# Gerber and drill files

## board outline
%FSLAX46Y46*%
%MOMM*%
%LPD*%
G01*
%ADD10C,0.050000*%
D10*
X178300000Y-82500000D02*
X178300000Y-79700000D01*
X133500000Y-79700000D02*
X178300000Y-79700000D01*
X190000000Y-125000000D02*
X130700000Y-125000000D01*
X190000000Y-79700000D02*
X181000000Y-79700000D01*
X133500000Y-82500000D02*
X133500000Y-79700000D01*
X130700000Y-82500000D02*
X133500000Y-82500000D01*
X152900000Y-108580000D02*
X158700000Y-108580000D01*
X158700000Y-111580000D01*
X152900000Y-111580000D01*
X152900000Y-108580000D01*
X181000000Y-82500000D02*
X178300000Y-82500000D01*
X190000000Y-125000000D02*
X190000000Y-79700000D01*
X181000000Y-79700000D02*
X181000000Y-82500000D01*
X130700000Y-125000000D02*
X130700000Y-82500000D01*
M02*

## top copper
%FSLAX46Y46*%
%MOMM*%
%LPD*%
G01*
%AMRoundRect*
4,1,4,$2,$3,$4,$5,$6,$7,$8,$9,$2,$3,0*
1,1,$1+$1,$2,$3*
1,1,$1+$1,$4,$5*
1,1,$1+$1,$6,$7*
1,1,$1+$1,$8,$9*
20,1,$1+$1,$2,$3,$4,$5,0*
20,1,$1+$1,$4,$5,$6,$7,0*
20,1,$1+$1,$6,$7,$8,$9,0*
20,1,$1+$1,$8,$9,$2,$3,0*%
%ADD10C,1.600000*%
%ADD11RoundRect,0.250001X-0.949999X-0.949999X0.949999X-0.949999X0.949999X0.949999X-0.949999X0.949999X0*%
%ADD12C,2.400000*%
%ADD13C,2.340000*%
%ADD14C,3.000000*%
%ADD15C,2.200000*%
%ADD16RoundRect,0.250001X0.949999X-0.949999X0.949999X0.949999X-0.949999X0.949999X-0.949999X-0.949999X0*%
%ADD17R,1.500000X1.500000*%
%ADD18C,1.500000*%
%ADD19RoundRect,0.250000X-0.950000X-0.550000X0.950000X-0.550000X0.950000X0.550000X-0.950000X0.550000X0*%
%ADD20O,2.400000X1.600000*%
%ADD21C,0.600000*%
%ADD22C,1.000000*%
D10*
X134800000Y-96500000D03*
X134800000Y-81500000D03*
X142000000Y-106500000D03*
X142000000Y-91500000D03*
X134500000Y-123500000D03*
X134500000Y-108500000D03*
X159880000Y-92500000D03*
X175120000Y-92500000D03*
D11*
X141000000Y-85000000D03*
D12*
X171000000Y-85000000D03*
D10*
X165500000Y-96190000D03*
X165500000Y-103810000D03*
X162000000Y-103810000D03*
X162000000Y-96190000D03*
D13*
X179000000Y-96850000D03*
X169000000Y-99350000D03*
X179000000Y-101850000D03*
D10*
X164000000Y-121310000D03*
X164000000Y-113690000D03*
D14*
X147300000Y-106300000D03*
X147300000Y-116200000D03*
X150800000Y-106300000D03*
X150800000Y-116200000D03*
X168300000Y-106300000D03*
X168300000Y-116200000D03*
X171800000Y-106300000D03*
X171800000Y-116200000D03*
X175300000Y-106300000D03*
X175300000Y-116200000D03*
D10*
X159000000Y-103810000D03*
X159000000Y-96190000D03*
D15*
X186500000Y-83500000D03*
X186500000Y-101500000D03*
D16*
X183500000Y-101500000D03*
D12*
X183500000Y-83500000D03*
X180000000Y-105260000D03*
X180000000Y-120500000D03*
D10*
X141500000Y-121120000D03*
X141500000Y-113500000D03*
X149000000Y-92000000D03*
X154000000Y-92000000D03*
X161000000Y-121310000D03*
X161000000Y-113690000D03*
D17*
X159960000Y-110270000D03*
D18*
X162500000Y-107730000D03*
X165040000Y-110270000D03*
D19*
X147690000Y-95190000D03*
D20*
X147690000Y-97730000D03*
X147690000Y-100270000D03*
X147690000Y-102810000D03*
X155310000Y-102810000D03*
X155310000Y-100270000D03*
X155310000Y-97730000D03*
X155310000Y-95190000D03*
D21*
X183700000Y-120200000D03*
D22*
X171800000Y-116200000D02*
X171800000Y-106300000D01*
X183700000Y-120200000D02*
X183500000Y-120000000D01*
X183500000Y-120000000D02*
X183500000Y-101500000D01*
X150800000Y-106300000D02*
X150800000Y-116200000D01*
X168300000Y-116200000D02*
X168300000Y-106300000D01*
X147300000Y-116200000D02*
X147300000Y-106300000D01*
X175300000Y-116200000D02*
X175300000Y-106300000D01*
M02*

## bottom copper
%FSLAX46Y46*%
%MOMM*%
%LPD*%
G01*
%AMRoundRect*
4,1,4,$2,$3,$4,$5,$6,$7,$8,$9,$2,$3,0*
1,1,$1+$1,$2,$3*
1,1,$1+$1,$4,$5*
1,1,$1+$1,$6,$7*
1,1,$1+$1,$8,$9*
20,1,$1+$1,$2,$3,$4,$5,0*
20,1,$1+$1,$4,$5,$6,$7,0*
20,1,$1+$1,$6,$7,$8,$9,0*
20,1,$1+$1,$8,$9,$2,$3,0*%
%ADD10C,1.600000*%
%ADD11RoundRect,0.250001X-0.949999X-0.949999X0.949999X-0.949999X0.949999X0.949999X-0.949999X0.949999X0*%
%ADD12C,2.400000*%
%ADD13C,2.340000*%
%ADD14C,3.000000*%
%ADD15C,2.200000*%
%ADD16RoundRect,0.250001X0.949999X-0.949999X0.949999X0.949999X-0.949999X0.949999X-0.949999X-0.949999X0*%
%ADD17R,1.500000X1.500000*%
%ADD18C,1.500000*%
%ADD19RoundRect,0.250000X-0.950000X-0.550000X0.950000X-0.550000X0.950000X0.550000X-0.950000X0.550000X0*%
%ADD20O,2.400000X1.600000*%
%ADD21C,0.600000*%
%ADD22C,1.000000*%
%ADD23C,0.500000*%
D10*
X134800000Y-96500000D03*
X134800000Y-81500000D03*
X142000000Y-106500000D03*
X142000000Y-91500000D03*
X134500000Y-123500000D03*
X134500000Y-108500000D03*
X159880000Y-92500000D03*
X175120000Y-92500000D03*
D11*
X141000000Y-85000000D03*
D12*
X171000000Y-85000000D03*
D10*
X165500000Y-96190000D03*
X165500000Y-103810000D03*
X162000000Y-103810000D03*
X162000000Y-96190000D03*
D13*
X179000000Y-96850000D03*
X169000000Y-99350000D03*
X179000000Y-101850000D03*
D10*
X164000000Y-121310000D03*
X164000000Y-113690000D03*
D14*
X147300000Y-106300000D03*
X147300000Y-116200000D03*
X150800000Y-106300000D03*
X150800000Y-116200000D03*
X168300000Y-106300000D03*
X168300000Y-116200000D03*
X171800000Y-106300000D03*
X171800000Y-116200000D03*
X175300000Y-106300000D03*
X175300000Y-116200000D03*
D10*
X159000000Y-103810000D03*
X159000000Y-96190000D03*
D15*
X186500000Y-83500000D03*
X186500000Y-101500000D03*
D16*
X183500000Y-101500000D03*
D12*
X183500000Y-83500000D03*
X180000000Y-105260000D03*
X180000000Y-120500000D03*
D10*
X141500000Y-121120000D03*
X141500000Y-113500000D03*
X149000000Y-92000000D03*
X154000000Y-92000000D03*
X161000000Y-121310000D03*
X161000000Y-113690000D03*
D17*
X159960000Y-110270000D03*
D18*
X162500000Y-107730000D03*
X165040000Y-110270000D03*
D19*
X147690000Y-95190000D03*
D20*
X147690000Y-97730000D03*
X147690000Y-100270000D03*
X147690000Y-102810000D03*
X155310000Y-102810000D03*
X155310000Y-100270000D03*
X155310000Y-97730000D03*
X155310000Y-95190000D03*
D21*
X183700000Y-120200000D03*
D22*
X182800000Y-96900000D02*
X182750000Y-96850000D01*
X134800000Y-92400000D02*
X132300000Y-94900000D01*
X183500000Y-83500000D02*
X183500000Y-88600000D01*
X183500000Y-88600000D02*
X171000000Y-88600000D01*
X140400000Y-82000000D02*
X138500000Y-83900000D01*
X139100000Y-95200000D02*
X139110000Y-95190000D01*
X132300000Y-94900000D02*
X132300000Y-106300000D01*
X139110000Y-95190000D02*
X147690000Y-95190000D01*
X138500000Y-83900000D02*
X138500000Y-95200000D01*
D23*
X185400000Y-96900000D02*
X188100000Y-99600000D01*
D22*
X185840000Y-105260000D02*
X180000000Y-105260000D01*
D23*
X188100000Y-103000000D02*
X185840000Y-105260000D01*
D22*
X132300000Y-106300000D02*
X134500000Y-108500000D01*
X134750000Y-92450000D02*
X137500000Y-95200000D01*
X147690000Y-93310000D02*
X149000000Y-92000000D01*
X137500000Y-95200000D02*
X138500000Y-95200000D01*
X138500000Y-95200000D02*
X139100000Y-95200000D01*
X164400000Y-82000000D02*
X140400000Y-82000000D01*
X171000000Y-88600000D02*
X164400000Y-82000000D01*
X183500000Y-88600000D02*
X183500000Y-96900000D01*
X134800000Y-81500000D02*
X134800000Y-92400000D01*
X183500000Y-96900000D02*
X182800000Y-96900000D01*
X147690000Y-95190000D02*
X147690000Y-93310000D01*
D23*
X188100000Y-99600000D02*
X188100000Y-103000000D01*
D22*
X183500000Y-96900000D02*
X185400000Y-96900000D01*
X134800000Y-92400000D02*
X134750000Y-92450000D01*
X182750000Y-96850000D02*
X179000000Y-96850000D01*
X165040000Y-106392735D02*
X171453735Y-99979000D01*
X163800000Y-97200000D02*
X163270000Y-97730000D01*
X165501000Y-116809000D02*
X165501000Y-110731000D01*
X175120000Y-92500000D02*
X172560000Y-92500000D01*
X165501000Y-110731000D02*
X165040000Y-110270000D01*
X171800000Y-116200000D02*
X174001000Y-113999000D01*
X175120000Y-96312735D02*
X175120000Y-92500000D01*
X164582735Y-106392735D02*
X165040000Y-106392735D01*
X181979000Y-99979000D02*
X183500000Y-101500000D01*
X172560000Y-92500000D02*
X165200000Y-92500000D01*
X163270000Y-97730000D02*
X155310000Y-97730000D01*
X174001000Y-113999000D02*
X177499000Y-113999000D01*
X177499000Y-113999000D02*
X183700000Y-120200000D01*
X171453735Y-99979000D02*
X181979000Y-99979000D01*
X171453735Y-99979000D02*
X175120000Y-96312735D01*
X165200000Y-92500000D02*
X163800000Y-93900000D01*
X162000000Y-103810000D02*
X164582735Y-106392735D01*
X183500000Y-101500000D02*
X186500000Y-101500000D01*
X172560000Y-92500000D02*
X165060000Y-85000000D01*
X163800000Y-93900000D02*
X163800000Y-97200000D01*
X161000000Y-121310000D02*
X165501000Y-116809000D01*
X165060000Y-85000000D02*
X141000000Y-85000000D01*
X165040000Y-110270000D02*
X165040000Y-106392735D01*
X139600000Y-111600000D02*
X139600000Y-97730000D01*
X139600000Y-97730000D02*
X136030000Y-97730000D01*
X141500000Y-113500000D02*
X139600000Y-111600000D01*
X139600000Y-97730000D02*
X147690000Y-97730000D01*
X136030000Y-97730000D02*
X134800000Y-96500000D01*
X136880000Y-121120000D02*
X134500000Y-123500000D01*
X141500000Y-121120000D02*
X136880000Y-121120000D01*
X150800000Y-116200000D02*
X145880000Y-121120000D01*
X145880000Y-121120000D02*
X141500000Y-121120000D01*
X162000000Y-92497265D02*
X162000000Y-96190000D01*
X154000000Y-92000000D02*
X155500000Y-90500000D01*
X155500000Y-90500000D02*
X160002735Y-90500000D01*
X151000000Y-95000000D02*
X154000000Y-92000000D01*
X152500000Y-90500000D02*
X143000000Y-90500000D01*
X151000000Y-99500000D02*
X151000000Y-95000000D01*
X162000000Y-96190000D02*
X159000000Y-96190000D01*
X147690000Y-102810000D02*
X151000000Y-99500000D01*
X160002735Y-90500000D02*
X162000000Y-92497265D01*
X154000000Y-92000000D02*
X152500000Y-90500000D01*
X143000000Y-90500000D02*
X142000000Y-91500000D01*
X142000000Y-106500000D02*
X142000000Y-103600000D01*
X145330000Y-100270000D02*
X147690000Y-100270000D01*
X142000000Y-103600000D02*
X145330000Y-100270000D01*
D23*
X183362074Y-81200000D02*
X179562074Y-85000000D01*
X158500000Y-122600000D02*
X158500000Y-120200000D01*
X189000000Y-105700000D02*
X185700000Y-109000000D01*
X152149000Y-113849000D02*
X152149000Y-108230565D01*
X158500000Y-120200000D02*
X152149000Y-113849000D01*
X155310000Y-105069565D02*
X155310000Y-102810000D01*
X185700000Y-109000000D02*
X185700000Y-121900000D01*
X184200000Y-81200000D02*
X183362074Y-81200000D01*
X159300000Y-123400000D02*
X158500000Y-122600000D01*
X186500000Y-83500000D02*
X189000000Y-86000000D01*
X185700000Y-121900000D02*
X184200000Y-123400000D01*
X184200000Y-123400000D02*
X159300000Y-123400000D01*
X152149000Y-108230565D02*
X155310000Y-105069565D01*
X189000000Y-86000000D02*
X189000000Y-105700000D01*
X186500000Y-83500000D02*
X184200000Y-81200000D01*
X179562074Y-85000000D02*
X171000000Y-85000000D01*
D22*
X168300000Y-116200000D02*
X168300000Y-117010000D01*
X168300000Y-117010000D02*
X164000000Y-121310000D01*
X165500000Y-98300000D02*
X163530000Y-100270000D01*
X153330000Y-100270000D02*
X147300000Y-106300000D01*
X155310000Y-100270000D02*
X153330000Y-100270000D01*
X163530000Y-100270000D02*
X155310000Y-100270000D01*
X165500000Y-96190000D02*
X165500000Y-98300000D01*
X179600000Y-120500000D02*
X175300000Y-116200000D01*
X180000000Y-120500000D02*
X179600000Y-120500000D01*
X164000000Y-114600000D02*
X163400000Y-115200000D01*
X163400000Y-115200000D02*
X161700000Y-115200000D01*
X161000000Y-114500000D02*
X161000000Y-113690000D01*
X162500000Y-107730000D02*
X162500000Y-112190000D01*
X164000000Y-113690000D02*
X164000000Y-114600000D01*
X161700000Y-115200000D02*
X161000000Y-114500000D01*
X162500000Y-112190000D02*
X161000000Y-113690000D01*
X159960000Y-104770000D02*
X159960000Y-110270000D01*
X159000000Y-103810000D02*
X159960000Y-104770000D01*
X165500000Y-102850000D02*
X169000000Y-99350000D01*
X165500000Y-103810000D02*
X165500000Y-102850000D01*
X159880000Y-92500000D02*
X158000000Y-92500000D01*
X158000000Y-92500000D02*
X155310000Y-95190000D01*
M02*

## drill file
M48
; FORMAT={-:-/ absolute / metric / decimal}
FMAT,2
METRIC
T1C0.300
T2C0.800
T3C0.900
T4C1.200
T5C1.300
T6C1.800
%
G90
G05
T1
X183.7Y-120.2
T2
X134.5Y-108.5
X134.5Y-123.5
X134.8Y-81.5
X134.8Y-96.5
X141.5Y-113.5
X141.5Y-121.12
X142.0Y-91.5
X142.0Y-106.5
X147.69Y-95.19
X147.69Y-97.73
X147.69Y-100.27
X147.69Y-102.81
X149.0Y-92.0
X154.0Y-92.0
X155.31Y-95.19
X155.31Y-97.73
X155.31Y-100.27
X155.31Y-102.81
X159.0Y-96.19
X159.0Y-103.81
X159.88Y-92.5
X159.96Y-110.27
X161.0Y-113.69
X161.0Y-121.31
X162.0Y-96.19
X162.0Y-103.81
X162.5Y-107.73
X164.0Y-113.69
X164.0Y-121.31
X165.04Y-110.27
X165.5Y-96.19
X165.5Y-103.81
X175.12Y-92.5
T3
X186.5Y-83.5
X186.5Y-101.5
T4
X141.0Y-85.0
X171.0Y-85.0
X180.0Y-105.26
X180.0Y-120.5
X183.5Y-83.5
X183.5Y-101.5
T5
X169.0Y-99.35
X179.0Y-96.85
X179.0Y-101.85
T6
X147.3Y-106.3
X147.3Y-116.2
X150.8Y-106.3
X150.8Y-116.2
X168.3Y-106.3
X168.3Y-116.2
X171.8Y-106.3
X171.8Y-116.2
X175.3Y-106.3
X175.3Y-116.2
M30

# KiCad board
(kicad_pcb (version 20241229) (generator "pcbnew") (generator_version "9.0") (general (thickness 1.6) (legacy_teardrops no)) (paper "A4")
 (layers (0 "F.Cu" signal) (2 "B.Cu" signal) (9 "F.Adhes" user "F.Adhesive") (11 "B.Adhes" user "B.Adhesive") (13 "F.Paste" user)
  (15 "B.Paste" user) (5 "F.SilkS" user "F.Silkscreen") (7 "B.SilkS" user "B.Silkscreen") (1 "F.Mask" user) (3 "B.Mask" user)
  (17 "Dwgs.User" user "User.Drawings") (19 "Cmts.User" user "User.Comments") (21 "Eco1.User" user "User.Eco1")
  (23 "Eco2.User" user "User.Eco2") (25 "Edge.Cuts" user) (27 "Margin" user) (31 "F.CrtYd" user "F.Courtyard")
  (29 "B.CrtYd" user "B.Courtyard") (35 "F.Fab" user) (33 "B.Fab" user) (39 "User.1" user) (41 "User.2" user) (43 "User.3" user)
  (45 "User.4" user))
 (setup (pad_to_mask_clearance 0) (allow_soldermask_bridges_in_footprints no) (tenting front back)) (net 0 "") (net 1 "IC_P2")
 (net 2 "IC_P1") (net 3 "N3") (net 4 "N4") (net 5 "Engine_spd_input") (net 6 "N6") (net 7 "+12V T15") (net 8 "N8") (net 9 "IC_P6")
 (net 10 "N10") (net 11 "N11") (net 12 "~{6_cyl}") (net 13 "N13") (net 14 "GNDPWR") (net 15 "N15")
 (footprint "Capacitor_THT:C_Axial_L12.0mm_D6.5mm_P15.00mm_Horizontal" (layer "F.Cu") (at 134.8 96.5 90)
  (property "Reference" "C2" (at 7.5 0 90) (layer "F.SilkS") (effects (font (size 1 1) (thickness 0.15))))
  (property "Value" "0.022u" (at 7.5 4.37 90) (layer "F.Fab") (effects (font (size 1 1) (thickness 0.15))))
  (pad "1" thru_hole circle (at 0 0 90) (size 1.6 1.6) (drill 0.8) (layers "*.Cu" "*.Mask") (remove_unused_layers no) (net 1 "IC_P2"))
  (pad "2" thru_hole circle (at 15 0 90) (size 1.6 1.6) (drill 0.8) (layers "*.Cu" "*.Mask") (remove_unused_layers no) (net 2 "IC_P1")))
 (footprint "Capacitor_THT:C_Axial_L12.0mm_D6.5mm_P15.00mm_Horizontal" (layer "F.Cu") (at 142 106.5 90)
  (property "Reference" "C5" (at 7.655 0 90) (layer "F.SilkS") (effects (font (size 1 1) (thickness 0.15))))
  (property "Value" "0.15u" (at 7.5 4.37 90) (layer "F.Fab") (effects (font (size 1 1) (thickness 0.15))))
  (pad "1" thru_hole circle (at 0 0 90) (size 1.6 1.6) (drill 0.8) (layers "*.Cu" "*.Mask") (remove_unused_layers no) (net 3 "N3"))
  (pad "2" thru_hole circle (at 15 0 90) (size 1.6 1.6) (drill 0.8) (layers "*.Cu" "*.Mask") (remove_unused_layers no) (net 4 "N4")))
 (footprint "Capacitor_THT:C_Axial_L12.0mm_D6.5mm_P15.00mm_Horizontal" (layer "F.Cu") (at 134.5 123.5 90)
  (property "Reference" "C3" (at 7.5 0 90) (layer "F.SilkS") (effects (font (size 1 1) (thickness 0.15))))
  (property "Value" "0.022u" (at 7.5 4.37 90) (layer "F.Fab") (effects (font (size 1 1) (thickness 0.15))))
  (pad "1" thru_hole circle (at 0 0 90) (size 1.6 1.6) (drill 0.8) (layers "*.Cu" "*.Mask") (remove_unused_layers no)
   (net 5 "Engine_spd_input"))
  (pad "2" thru_hole circle (at 15 0 90) (size 1.6 1.6) (drill 0.8) (layers "*.Cu" "*.Mask") (remove_unused_layers no) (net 2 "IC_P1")))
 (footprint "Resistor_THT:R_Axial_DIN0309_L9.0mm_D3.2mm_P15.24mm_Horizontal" (layer "F.Cu") (at 159.88 92.5)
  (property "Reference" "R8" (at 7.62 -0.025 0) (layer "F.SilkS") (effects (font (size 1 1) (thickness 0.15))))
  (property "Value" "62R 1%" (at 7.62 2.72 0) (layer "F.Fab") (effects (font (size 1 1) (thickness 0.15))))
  (pad "1" thru_hole circle (at 0 0) (size 1.6 1.6) (drill 0.8) (layers "*.Cu" "*.Mask") (remove_unused_layers no) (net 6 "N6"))
  (pad "2" thru_hole circle (at 15.24 0) (size 1.6 1.6) (drill 0.8) (layers "*.Cu" "*.Mask") (remove_unused_layers no) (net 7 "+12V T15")))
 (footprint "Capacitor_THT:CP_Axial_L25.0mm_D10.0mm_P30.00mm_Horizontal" (layer "F.Cu") (at 141 85)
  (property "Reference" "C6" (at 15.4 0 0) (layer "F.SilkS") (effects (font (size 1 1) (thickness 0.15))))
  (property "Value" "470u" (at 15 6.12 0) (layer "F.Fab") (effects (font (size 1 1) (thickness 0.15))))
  (pad "1" thru_hole roundrect (at 0 0) (size 2.4 2.4) (drill 1.2) (layers "*.Cu" "*.Mask") (remove_unused_layers no)
   (roundrect_rratio 0.104167) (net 7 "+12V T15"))
  (pad "2" thru_hole circle (at 30 0) (size 2.4 2.4) (drill 1.2) (layers "*.Cu" "*.Mask") (remove_unused_layers no) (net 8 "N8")))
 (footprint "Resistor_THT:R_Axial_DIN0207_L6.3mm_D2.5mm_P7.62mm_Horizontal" (layer "F.Cu") (at 165.5 96.19 -90)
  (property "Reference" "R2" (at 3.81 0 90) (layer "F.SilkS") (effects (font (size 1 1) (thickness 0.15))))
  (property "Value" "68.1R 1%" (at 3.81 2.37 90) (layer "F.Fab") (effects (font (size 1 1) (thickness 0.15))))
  (pad "1" thru_hole circle (at 0 0 270) (size 1.6 1.6) (drill 0.8) (layers "*.Cu" "*.Mask") (remove_unused_layers no) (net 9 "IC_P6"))
  (pad "2" thru_hole circle (at 7.62 0 270) (size 1.6 1.6) (drill 0.8) (layers "*.Cu" "*.Mask") (remove_unused_layers no) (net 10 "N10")))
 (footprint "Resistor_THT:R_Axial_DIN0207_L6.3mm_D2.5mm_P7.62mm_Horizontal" (layer "F.Cu") (at 162 103.81 90)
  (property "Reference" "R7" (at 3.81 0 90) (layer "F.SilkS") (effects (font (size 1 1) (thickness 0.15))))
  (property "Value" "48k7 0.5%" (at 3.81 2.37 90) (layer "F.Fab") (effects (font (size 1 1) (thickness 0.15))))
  (pad "1" thru_hole circle (at 0 0 90) (size 1.6 1.6) (drill 0.8) (layers "*.Cu" "*.Mask") (remove_unused_layers no) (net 7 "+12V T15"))
  (pad "2" thru_hole circle (at 7.62 0 90) (size 1.6 1.6) (drill 0.8) (layers "*.Cu" "*.Mask") (remove_unused_layers no) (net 4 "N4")))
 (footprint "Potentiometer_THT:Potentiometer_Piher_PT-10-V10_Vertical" (layer "F.Cu") (at 179 96.85 180)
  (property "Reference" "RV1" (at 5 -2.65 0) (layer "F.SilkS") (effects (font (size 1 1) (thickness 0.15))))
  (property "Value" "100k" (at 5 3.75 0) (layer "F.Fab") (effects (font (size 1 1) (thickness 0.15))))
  (pad "1" thru_hole circle (at 0 0 180) (size 2.34 2.34) (drill 1.3) (layers "*.Cu" "*.Mask") (remove_unused_layers no) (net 2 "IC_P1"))
  (pad "2" thru_hole circle (at 10 -2.5 180) (size 2.34 2.34) (drill 1.3) (layers "*.Cu" "*.Mask") (remove_unused_layers no) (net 10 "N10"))
  (pad "3" thru_hole circle (at 0 -5 180) (size 2.34 2.34) (drill 1.3) (layers "*.Cu" "*.Mask") (remove_unused_layers no) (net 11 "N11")))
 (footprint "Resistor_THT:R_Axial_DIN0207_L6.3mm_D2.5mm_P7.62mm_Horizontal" (layer "F.Cu") (at 164 121.31 90)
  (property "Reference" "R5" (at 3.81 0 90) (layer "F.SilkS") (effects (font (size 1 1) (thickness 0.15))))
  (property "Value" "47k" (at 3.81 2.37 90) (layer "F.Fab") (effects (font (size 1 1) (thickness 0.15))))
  (pad "1" thru_hole circle (at 0 0 90) (size 1.6 1.6) (drill 0.8) (layers "*.Cu" "*.Mask") (remove_unused_layers no) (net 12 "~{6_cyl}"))
  (pad "2" thru_hole circle (at 7.62 0 90) (size 1.6 1.6) (drill 0.8) (layers "*.Cu" "*.Mask") (remove_unused_layers no) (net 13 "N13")))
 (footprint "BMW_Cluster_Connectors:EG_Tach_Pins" (layer "F.Cu") (at 147.3 106.3)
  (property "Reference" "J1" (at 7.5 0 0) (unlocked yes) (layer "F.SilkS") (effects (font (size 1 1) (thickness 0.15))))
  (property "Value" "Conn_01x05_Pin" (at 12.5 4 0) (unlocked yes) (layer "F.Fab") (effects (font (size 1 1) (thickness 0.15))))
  (pad "1" thru_hole circle (at 0 0 270) (size 3 3) (drill 1.8) (layers "*.Cu" "*.Mask") (remove_unused_layers no) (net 9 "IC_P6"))
  (pad "1" thru_hole circle (at 0 9.9 270) (size 3 3) (drill 1.8) (layers "*.Cu" "*.Mask") (remove_unused_layers no) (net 9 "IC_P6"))
  (pad "2" thru_hole circle (at 3.5 0 270) (size 3 3) (drill 1.8) (layers "*.Cu" "*.Mask") (remove_unused_layers no)
   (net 5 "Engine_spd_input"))
  (pad "2" thru_hole circle (at 3.5 9.9 270) (size 3 3) (drill 1.8) (layers "*.Cu" "*.Mask") (remove_unused_layers no)
   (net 5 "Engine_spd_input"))
  (pad "3" thru_hole circle (at 21 0 270) (size 3 3) (drill 1.8) (layers "*.Cu" "*.Mask") (remove_unused_layers no) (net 12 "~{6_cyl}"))
  (pad "3" thru_hole circle (at 21 9.9 270) (size 3 3) (drill 1.8) (layers "*.Cu" "*.Mask") (remove_unused_layers no) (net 12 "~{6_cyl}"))
  (pad "4" thru_hole circle (at 24.5 0 270) (size 3 3) (drill 1.8) (layers "*.Cu" "*.Mask") (remove_unused_layers no) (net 7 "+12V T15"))
  (pad "4" thru_hole circle (at 24.5 9.9 270) (size 3 3) (drill 1.8) (layers "*.Cu" "*.Mask") (remove_unused_layers no) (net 7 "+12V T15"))
  (pad "5" thru_hole circle (at 28 0 270) (size 3 3) (drill 1.8) (layers "*.Cu" "*.Mask") (remove_unused_layers no) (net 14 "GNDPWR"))
  (pad "5" thru_hole circle (at 28 9.9 270) (size 3 3) (drill 1.8) (layers "*.Cu" "*.Mask") (remove_unused_layers no) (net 14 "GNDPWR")))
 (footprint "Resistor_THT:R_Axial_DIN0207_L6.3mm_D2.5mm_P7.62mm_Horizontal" (layer "F.Cu") (at 159 103.81 90)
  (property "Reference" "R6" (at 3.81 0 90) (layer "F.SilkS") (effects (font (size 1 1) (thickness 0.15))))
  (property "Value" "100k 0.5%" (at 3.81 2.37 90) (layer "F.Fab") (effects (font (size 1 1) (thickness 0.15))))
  (pad "1" thru_hole circle (at 0 0 90) (size 1.6 1.6) (drill 0.8) (layers "*.Cu" "*.Mask") (remove_unused_layers no) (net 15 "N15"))
  (pad "2" thru_hole circle (at 7.62 0 90) (size 1.6 1.6) (drill 0.8) (layers "*.Cu" "*.Mask") (remove_unused_layers no) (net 4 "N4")))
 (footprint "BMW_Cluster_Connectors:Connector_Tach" (layer "F.Cu") (at 186.5 83.5)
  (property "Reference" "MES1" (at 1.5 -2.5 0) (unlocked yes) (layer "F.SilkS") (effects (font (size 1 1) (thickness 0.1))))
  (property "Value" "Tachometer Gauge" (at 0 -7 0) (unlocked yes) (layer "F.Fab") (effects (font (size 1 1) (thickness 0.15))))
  (pad "1" thru_hole circle (at 0 0) (size 2.2 2.2) (drill 0.9) (layers "*.Cu" "*.Mask") (remove_unused_layers no) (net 8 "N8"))
  (pad "2" thru_hole circle (at 0 18) (size 2.2 2.2) (drill 0.9) (layers "*.Cu" "*.Mask") (remove_unused_layers no) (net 7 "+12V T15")))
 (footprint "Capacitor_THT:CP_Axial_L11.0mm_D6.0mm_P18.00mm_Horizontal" (layer "F.Cu") (at 183.5 101.5 90)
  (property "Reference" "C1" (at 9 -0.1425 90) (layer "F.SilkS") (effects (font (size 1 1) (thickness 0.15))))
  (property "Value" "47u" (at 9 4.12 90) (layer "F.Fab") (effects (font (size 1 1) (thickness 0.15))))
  (pad "1" thru_hole roundrect (at 0 0 90) (size 2.4 2.4) (drill 1.2) (layers "*.Cu" "*.Mask") (remove_unused_layers no)
   (roundrect_rratio 0.104167) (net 7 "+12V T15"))
  (pad "2" thru_hole circle (at 18 0 90) (size 2.4 2.4) (drill 1.2) (layers "*.Cu" "*.Mask") (remove_unused_layers no) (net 2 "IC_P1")))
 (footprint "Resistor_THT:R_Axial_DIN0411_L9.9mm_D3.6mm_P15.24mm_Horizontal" (layer "F.Cu") (at 180 105.26 -90)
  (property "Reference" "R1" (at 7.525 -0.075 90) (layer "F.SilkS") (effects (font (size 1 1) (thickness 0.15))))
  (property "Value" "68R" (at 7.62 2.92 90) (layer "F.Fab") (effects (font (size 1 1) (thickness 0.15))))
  (pad "1" thru_hole circle (at 0 0 270) (size 2.4 2.4) (drill 1.2) (layers "*.Cu" "*.Mask") (remove_unused_layers no) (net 2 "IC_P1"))
  (pad "2" thru_hole circle (at 15.24 0 270) (size 2.4 2.4) (drill 1.2) (layers "*.Cu" "*.Mask") (remove_unused_layers no) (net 14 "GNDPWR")))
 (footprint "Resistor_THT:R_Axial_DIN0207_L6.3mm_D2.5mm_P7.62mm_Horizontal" (layer "F.Cu") (at 141.5 121.12 90)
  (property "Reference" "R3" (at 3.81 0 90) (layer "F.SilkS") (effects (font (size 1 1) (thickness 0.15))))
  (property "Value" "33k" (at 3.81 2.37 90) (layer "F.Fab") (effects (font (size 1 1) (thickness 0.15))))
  (pad "1" thru_hole circle (at 0 0 90) (size 1.6 1.6) (drill 0.8) (layers "*.Cu" "*.Mask") (remove_unused_layers no)
   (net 5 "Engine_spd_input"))
  (pad "2" thru_hole circle (at 7.62 0 90) (size 1.6 1.6) (drill 0.8) (layers "*.Cu" "*.Mask") (remove_unused_layers no) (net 1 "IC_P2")))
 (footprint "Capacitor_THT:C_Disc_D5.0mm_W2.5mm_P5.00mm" (layer "F.Cu") (at 149 92)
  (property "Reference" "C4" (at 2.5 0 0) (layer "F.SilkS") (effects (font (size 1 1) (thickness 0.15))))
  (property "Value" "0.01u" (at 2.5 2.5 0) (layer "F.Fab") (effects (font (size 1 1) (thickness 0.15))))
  (pad "1" thru_hole circle (at 0 0) (size 1.6 1.6) (drill 0.8) (layers "*.Cu" "*.Mask") (remove_unused_layers no) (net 2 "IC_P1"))
  (pad "2" thru_hole circle (at 5 0) (size 1.6 1.6) (drill 0.8) (layers "*.Cu" "*.Mask") (remove_unused_layers no) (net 4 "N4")))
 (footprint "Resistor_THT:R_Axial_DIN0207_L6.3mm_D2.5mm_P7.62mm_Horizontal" (layer "F.Cu") (at 161 121.31 90)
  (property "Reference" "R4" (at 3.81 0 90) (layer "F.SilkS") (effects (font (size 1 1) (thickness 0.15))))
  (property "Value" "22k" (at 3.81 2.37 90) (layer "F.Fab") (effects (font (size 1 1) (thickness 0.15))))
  (pad "1" thru_hole circle (at 0 0 90) (size 1.6 1.6) (drill 0.8) (layers "*.Cu" "*.Mask") (remove_unused_layers no) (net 7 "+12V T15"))
  (pad "2" thru_hole circle (at 7.62 0 90) (size 1.6 1.6) (drill 0.8) (layers "*.Cu" "*.Mask") (remove_unused_layers no) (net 13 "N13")))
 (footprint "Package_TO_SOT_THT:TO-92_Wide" (layer "F.Cu") (at 159.96 110.27)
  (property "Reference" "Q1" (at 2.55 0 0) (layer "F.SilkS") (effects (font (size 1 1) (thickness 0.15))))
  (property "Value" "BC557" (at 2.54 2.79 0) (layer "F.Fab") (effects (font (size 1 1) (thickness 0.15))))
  (pad "1" thru_hole rect (at 0 0) (size 1.5 1.5) (drill 0.8) (layers "*.Cu" "*.Mask") (remove_unused_layers no) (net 15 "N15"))
  (pad "2" thru_hole circle (at 2.54 -2.54) (size 1.5 1.5) (drill 0.8) (layers "*.Cu" "*.Mask") (remove_unused_layers no) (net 13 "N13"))
  (pad "3" thru_hole circle (at 5.08 0) (size 1.5 1.5) (drill 0.8) (layers "*.Cu" "*.Mask") (remove_unused_layers no) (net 7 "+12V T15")))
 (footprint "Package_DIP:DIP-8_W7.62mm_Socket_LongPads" (layer "F.Cu") (at 147.69 95.19)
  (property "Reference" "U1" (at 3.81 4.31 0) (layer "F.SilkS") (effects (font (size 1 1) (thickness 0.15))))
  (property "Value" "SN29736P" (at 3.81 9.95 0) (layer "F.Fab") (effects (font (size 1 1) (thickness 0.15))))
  (pad "1" thru_hole roundrect (at 0 0) (size 2.4 1.6) (drill 0.8) (layers "*.Cu" "*.Mask") (remove_unused_layers no)
   (roundrect_rratio 0.15625) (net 2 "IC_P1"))
  (pad "2" thru_hole oval (at 0 2.54) (size 2.4 1.6) (drill 0.8) (layers "*.Cu" "*.Mask") (remove_unused_layers no) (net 1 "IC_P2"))
  (pad "3" thru_hole oval (at 0 5.08) (size 2.4 1.6) (drill 0.8) (layers "*.Cu" "*.Mask") (remove_unused_layers no) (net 3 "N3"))
  (pad "4" thru_hole oval (at 0 7.62) (size 2.4 1.6) (drill 0.8) (layers "*.Cu" "*.Mask") (remove_unused_layers no) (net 4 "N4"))
  (pad "5" thru_hole oval (at 7.62 7.62) (size 2.4 1.6) (drill 0.8) (layers "*.Cu" "*.Mask") (remove_unused_layers no) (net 8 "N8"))
  (pad "6" thru_hole oval (at 7.62 5.08) (size 2.4 1.6) (drill 0.8) (layers "*.Cu" "*.Mask") (remove_unused_layers no) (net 9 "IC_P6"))
  (pad "7" thru_hole oval (at 7.62 2.54) (size 2.4 1.6) (drill 0.8) (layers "*.Cu" "*.Mask") (remove_unused_layers no) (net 7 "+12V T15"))
  (pad "8" thru_hole oval (at 7.62 0) (size 2.4 1.6) (drill 0.8) (layers "*.Cu" "*.Mask") (remove_unused_layers no) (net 6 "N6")))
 (gr_line (start 178.3 82.5) (end 178.3 79.7) (stroke (width 0.05) (type solid)) (layer "Edge.Cuts"))
 (gr_line (start 133.5 79.7) (end 178.3 79.7) (stroke (width 0.05) (type default)) (layer "Edge.Cuts"))
 (gr_line (start 190 125) (end 130.7 125) (stroke (width 0.05) (type solid)) (layer "Edge.Cuts"))
 (gr_line (start 190 79.7) (end 181 79.7) (stroke (width 0.05) (type solid)) (layer "Edge.Cuts"))
 (gr_line (start 133.5 82.5) (end 133.5 79.7) (stroke (width 0.05) (type solid)) (layer "Edge.Cuts"))
 (gr_line (start 130.7 82.5) (end 133.5 82.5) (stroke (width 0.05) (type solid)) (layer "Edge.Cuts"))
 (gr_rect (start 152.9 111.58) (end 158.7 108.58) (stroke (width 0.05) (type solid)) (fill no) (layer "Edge.Cuts"))
 (gr_line (start 181 82.5) (end 178.3 82.5) (stroke (width 0.05) (type solid)) (layer "Edge.Cuts"))
 (gr_line (start 190 125) (end 190 79.7) (stroke (width 0.05) (type solid)) (layer "Edge.Cuts"))
 (gr_line (start 181 79.7) (end 181 82.5) (stroke (width 0.05) (type default)) (layer "Edge.Cuts"))
 (gr_line (start 130.7 125) (end 130.7 82.5) (stroke (width 0.05) (type solid)) (layer "Edge.Cuts"))
 (segment (start 182.8 96.9) (end 182.75 96.85) (width 1) (layer "B.Cu") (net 2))
 (segment (start 134.8 92.4) (end 132.3 94.9) (width 1) (layer "B.Cu") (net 2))
 (segment (start 183.5 83.5) (end 183.5 88.6) (width 1) (layer "B.Cu") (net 2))
 (segment (start 183.5 88.6) (end 171 88.6) (width 1) (layer "B.Cu") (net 2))
 (segment (start 140.4 82) (end 138.5 83.9) (width 1) (layer "B.Cu") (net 2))
 (segment (start 139.1 95.2) (end 139.11 95.19) (width 1) (layer "B.Cu") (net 2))
 (segment (start 132.3 94.9) (end 132.3 106.3) (width 1) (layer "B.Cu") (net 2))
 (segment (start 139.11 95.19) (end 147.69 95.19) (width 1) (layer "B.Cu") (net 2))
 (segment (start 138.5 83.9) (end 138.5 95.2) (width 1) (layer "B.Cu") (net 2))
 (segment (start 185.4 96.9) (end 188.1 99.6) (width 0.5) (layer "B.Cu") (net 2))
 (segment (start 185.84 105.26) (end 180 105.26) (width 1) (layer "B.Cu") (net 2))
 (segment (start 188.1 103) (end 185.84 105.26) (width 0.5) (layer "B.Cu") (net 2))
 (segment (start 132.3 106.3) (end 134.5 108.5) (width 1) (layer "B.Cu") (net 2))
 (segment (start 134.75 92.45) (end 137.5 95.2) (width 1) (layer "B.Cu") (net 2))
 (segment (start 147.69 93.31) (end 149 92) (width 1) (layer "B.Cu") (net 2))
 (segment (start 137.5 95.2) (end 138.5 95.2) (width 1) (layer "B.Cu") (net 2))
 (segment (start 138.5 95.2) (end 139.1 95.2) (width 1) (layer "B.Cu") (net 2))
 (segment (start 164.4 82) (end 140.4 82) (width 1) (layer "B.Cu") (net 2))
 (segment (start 171 88.6) (end 164.4 82) (width 1) (layer "B.Cu") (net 2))
 (segment (start 183.5 88.6) (end 183.5 96.9) (width 1) (layer "B.Cu") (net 2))
 (segment (start 134.8 81.5) (end 134.8 92.4) (width 1) (layer "B.Cu") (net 2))
 (segment (start 183.5 96.9) (end 182.8 96.9) (width 1) (layer "B.Cu") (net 2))
 (segment (start 147.69 95.19) (end 147.69 93.31) (width 1) (layer "B.Cu") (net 2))
 (segment (start 188.1 99.6) (end 188.1 103) (width 0.5) (layer "B.Cu") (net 2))
 (segment (start 183.5 96.9) (end 185.4 96.9) (width 1) (layer "B.Cu") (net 2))
 (segment (start 134.8 92.4) (end 134.75 92.45) (width 1) (layer "B.Cu") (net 2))
 (segment (start 182.75 96.85) (end 179 96.85) (width 1) (layer "B.Cu") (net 2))
 (segment (start 171.8 116.2) (end 171.8 106.3) (width 1) (layer "F.Cu") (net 7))
 (segment (start 183.7 120.2) (end 183.5 120) (width 1) (layer "F.Cu") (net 7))
 (segment (start 183.5 120) (end 183.5 101.5) (width 1) (layer "F.Cu") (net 7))
 (via (at 183.7 120.2) (size 0.6) (drill 0.3) (layers "F.Cu" "B.Cu") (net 7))
 (segment (start 165.04 106.392735) (end 171.453735 99.979) (width 1) (layer "B.Cu") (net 7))
 (segment (start 163.8 97.2) (end 163.27 97.73) (width 1) (layer "B.Cu") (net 7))
 (segment (start 165.501 116.809) (end 165.501 110.731) (width 1) (layer "B.Cu") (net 7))
 (segment (start 175.12 92.5) (end 172.56 92.5) (width 1) (layer "B.Cu") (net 7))
 (segment (start 165.501 110.731) (end 165.04 110.27) (width 1) (layer "B.Cu") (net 7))
 (segment (start 171.8 116.2) (end 174.001 113.999) (width 1) (layer "B.Cu") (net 7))
 (segment (start 175.12 96.312735) (end 175.12 92.5) (width 1) (layer "B.Cu") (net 7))
 (segment (start 164.582735 106.392735) (end 165.04 106.392735) (width 1) (layer "B.Cu") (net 7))
 (segment (start 181.979 99.979) (end 183.5 101.5) (width 1) (layer "B.Cu") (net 7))
 (segment (start 172.56 92.5) (end 165.2 92.5) (width 1) (layer "B.Cu") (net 7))
 (segment (start 163.27 97.73) (end 155.31 97.73) (width 1) (layer "B.Cu") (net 7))
 (segment (start 174.001 113.999) (end 177.499 113.999) (width 1) (layer "B.Cu") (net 7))
 (segment (start 177.499 113.999) (end 183.7 120.2) (width 1) (layer "B.Cu") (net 7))
 (segment (start 171.453735 99.979) (end 181.979 99.979) (width 1) (layer "B.Cu") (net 7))
 (segment (start 171.453735 99.979) (end 175.12 96.312735) (width 1) (layer "B.Cu") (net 7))
 (segment (start 165.2 92.5) (end 163.8 93.9) (width 1) (layer "B.Cu") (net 7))
 (segment (start 162 103.81) (end 164.582735 106.392735) (width 1) (layer "B.Cu") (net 7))
 (segment (start 183.5 101.5) (end 186.5 101.5) (width 1) (layer "B.Cu") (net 7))
 (segment (start 172.56 92.5) (end 165.06 85) (width 1) (layer "B.Cu") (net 7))
 (segment (start 163.8 93.9) (end 163.8 97.2) (width 1) (layer "B.Cu") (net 7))
 (segment (start 161 121.31) (end 165.501 116.809) (width 1) (layer "B.Cu") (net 7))
 (segment (start 165.06 85) (end 141 85) (width 1) (layer "B.Cu") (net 7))
 (segment (start 165.04 110.27) (end 165.04 106.392735) (width 1) (layer "B.Cu") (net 7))
 (segment (start 139.6 111.6) (end 139.6 97.73) (width 1) (layer "B.Cu") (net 1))
 (segment (start 139.6 97.73) (end 136.03 97.73) (width 1) (layer "B.Cu") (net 1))
 (segment (start 141.5 113.5) (end 139.6 111.6) (width 1) (layer "B.Cu") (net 1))
 (segment (start 139.6 97.73) (end 147.69 97.73) (width 1) (layer "B.Cu") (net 1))
 (segment (start 136.03 97.73) (end 134.8 96.5) (width 1) (layer "B.Cu") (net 1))
 (segment (start 150.8 106.3) (end 150.8 116.2) (width 1) (layer "F.Cu") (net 5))
 (segment (start 136.88 121.12) (end 134.5 123.5) (width 1) (layer "B.Cu") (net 5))
 (segment (start 141.5 121.12) (end 136.88 121.12) (width 1) (layer "B.Cu") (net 5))
 (segment (start 150.8 116.2) (end 145.88 121.12) (width 1) (layer "B.Cu") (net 5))
 (segment (start 145.88 121.12) (end 141.5 121.12) (width 1) (layer "B.Cu") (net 5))
 (segment (start 162 92.497265) (end 162 96.19) (width 1) (layer "B.Cu") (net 4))
 (segment (start 154 92) (end 155.5 90.5) (width 1) (layer "B.Cu") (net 4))
 (segment (start 155.5 90.5) (end 160.002735 90.5) (width 1) (layer "B.Cu") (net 4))
 (segment (start 151 95) (end 154 92) (width 1) (layer "B.Cu") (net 4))
 (segment (start 152.5 90.5) (end 143 90.5) (width 1) (layer "B.Cu") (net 4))
 (segment (start 151 99.5) (end 151 95) (width 1) (layer "B.Cu") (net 4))
 (segment (start 162 96.19) (end 159 96.19) (width 1) (layer "B.Cu") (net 4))
 (segment (start 147.69 102.81) (end 151 99.5) (width 1) (layer "B.Cu") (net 4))
 (segment (start 160.002735 90.5) (end 162 92.497265) (width 1) (layer "B.Cu") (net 4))
 (segment (start 154 92) (end 152.5 90.5) (width 1) (layer "B.Cu") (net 4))
 (segment (start 143 90.5) (end 142 91.5) (width 1) (layer "B.Cu") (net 4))
 (segment (start 142 106.5) (end 142 103.6) (width 1) (layer "B.Cu") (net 3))
 (segment (start 145.33 100.27) (end 147.69 100.27) (width 1) (layer "B.Cu") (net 3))
 (segment (start 142 103.6) (end 145.33 100.27) (width 1) (layer "B.Cu") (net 3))
 (segment (start 183.362074 81.2) (end 179.562074 85) (width 0.5) (layer "B.Cu") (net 8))
 (segment (start 158.5 122.6) (end 158.5 120.2) (width 0.5) (layer "B.Cu") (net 8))
 (segment (start 189 105.7) (end 185.7 109) (width 0.5) (layer "B.Cu") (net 8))
 (segment (start 152.149 113.849) (end 152.149 108.230565) (width 0.5) (layer "B.Cu") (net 8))
 (segment (start 158.5 120.2) (end 152.149 113.849) (width 0.5) (layer "B.Cu") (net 8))
 (segment (start 155.31 105.069565) (end 155.31 102.81) (width 0.5) (layer "B.Cu") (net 8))
 (segment (start 185.7 109) (end 185.7 121.9) (width 0.5) (layer "B.Cu") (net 8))
 (segment (start 184.2 81.2) (end 183.362074 81.2) (width 0.5) (layer "B.Cu") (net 8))
 (segment (start 159.3 123.4) (end 158.5 122.6) (width 0.5) (layer "B.Cu") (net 8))
 (segment (start 186.5 83.5) (end 189 86) (width 0.5) (layer "B.Cu") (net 8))
 (segment (start 185.7 121.9) (end 184.2 123.4) (width 0.5) (layer "B.Cu") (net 8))
 (segment (start 184.2 123.4) (end 159.3 123.4) (width 0.5) (layer "B.Cu") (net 8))
 (segment (start 152.149 108.230565) (end 155.31 105.069565) (width 0.5) (layer "B.Cu") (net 8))
 (segment (start 189 86) (end 189 105.7) (width 0.5) (layer "B.Cu") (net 8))
 (segment (start 186.5 83.5) (end 184.2 81.2) (width 0.5) (layer "B.Cu") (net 8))
 (segment (start 179.562074 85) (end 171 85) (width 0.5) (layer "B.Cu") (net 8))
 (segment (start 168.3 116.2) (end 168.3 106.3) (width 1) (layer "F.Cu") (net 12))
 (segment (start 168.3 116.2) (end 168.3 117.01) (width 1) (layer "B.Cu") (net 12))
 (segment (start 168.3 117.01) (end 164 121.31) (width 1) (layer "B.Cu") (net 12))
 (segment (start 147.3 116.2) (end 147.3 106.3) (width 1) (layer "F.Cu") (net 9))
 (segment (start 165.5 98.3) (end 163.53 100.27) (width 1) (layer "B.Cu") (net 9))
 (segment (start 153.33 100.27) (end 147.3 106.3) (width 1) (layer "B.Cu") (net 9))
 (segment (start 155.31 100.27) (end 153.33 100.27) (width 1) (layer "B.Cu") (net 9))
 (segment (start 163.53 100.27) (end 155.31 100.27) (width 1) (layer "B.Cu") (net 9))
 (segment (start 165.5 96.19) (end 165.5 98.3) (width 1) (layer "B.Cu") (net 9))
 (segment (start 175.3 116.2) (end 175.3 106.3) (width 1) (layer "F.Cu") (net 14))
 (segment (start 179.6 120.5) (end 175.3 116.2) (width 1) (layer "B.Cu") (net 14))
 (segment (start 180 120.5) (end 179.6 120.5) (width 1) (layer "B.Cu") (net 14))
 (segment (start 164 114.6) (end 163.4 115.2) (width 1) (layer "B.Cu") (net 13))
 (segment (start 163.4 115.2) (end 161.7 115.2) (width 1) (layer "B.Cu") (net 13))
 (segment (start 161 114.5) (end 161 113.69) (width 1) (layer "B.Cu") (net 13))
 (segment (start 162.5 107.73) (end 162.5 112.19) (width 1) (layer "B.Cu") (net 13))
 (segment (start 164 113.69) (end 164 114.6) (width 1) (layer "B.Cu") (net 13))
 (segment (start 161.7 115.2) (end 161 114.5) (width 1) (layer "B.Cu") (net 13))
 (segment (start 162.5 112.19) (end 161 113.69) (width 1) (layer "B.Cu") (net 13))
 (segment (start 159.96 104.77) (end 159.96 110.27) (width 1) (layer "B.Cu") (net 15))
 (segment (start 159 103.81) (end 159.96 104.77) (width 1) (layer "B.Cu") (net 15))
 (segment (start 165.5 102.85) (end 169 99.35) (width 1) (layer "B.Cu") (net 10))
 (segment (start 165.5 103.81) (end 165.5 102.85) (width 1) (layer "B.Cu") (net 10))
 (segment (start 159.88 92.5) (end 158 92.5) (width 1) (layer "B.Cu") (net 6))
 (segment (start 158 92.5) (end 155.31 95.19) (width 1) (layer "B.Cu") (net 6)))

